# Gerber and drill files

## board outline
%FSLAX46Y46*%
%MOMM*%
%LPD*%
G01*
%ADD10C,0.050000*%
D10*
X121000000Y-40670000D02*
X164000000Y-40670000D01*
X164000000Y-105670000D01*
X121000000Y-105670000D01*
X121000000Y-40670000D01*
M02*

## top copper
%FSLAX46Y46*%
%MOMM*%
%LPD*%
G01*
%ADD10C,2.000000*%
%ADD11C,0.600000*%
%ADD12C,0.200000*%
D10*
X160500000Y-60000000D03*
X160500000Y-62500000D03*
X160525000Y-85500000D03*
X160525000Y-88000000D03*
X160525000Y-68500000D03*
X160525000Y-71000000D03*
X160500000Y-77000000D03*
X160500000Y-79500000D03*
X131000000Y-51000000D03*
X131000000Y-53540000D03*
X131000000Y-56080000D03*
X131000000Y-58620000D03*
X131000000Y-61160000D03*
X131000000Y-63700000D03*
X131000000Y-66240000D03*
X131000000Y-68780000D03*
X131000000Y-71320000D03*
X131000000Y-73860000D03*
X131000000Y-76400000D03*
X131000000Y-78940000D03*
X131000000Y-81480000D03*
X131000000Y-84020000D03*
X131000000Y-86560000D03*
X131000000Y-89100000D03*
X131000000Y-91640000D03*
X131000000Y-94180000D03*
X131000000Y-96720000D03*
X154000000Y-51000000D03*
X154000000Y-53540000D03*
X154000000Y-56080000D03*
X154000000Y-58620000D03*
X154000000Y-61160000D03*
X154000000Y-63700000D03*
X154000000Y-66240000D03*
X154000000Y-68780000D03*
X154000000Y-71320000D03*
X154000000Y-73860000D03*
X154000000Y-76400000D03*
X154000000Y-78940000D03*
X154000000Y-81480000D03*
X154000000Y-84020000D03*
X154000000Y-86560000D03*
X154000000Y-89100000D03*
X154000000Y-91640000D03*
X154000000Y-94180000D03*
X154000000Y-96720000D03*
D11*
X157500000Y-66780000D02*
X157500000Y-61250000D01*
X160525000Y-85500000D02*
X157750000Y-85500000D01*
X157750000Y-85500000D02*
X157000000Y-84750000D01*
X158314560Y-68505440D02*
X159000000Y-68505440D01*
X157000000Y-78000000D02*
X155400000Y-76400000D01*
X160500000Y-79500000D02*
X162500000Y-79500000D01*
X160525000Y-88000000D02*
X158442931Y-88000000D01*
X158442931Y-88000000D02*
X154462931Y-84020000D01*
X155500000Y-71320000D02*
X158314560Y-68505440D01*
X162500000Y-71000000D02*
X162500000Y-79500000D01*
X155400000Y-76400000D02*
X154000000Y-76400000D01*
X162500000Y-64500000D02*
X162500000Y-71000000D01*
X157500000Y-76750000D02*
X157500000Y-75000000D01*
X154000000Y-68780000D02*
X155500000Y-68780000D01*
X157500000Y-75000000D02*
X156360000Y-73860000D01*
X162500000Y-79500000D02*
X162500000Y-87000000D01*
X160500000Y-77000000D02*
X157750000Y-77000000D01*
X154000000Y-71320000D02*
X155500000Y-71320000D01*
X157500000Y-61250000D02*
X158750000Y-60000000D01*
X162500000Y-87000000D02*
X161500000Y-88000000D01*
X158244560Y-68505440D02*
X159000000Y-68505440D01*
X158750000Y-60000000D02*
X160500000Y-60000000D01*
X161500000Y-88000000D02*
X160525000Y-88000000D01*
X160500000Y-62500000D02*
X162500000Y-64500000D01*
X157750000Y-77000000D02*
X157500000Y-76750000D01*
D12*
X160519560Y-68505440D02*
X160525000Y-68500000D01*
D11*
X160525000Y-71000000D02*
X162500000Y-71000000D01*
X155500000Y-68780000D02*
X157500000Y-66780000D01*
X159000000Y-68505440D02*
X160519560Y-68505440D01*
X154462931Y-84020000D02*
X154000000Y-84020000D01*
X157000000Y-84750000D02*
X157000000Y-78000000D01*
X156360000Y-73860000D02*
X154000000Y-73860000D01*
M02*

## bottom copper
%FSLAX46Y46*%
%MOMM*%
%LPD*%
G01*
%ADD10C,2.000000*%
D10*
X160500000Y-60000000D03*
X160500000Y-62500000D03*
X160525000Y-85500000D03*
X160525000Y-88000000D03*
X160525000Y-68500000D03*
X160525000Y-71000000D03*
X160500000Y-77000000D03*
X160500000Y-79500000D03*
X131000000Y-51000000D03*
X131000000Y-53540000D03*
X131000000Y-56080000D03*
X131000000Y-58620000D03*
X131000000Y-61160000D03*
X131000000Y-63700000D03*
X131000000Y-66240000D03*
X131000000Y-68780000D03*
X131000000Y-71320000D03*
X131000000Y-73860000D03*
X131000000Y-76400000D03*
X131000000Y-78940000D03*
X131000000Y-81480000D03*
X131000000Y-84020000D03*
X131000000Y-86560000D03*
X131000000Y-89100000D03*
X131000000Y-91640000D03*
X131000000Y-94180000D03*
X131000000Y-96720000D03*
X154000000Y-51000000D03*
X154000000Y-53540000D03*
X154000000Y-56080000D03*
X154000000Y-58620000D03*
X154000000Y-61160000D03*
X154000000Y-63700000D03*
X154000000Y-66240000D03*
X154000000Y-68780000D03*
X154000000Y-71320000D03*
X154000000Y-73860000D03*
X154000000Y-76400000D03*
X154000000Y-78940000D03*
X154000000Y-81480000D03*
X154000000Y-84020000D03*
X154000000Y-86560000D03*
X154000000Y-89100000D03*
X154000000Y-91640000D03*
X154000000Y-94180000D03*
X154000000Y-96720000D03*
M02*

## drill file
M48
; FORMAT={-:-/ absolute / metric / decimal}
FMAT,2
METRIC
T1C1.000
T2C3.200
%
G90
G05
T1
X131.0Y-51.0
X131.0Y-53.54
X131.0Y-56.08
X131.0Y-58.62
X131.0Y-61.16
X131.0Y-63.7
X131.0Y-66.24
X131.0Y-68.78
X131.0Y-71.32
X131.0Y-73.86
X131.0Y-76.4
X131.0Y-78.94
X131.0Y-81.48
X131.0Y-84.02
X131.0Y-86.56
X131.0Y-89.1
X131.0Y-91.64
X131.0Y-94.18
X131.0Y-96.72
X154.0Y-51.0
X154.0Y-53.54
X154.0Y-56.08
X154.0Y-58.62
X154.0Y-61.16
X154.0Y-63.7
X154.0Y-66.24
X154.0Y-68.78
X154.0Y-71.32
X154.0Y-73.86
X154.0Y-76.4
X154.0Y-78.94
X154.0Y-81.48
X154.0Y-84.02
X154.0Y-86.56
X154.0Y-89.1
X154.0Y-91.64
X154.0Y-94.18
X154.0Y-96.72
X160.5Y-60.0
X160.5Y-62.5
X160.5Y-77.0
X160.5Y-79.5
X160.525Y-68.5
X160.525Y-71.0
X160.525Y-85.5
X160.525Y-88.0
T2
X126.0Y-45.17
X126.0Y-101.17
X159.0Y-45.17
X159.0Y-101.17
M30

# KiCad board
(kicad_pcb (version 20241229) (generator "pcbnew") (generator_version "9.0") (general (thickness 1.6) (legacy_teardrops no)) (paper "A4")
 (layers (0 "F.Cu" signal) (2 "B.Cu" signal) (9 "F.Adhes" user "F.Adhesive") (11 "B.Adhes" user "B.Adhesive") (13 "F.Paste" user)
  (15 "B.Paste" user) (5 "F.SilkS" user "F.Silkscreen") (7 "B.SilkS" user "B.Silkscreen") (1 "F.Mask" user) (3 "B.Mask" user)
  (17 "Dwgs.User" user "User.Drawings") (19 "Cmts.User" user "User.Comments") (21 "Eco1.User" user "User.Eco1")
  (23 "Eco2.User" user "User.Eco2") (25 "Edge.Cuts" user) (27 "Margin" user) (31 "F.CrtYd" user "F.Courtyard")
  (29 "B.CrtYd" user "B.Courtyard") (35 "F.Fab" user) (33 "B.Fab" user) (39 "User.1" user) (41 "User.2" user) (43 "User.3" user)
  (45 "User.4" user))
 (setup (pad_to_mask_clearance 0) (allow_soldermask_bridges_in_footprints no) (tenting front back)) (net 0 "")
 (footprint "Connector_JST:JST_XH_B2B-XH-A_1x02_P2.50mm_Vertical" (layer "F.Cu") (at 160.5 60 -90)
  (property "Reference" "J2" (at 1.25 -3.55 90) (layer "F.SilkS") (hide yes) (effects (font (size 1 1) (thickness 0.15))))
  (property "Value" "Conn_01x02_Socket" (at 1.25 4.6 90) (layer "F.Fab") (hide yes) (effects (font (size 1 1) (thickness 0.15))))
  (pad "1" thru_hole circle (at 0 0 270) (size 2 2) (drill 1) (layers "*.Cu" "*.Mask") (remove_unused_layers no))
  (pad "2" thru_hole circle (at 2.5 0 270) (size 2 2) (drill 1) (layers "*.Cu" "*.Mask") (remove_unused_layers no)))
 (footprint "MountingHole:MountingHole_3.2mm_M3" (layer "F.Cu") (at 126 101.17)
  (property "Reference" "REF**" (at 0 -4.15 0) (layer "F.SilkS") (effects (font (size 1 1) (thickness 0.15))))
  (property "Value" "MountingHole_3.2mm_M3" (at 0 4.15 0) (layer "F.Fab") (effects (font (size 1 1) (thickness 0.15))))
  (pad "" np_thru_hole circle (at 0 0) (size 3.2 3.2) (drill 3.2) (layers "*.Cu" "*.Mask")))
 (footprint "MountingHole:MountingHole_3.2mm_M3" (layer "F.Cu") (at 159 45.17)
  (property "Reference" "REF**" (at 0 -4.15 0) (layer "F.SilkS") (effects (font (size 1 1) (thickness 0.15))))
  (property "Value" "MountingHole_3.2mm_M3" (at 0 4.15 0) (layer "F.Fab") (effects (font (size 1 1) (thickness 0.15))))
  (pad "" np_thru_hole circle (at 0 0) (size 3.2 3.2) (drill 3.2) (layers "*.Cu" "*.Mask")))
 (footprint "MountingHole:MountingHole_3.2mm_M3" (layer "F.Cu") (at 159 101.17)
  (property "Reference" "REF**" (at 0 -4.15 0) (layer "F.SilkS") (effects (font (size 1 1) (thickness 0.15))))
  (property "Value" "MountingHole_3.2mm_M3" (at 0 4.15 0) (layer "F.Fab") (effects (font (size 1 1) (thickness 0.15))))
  (pad "" np_thru_hole circle (at 0 0) (size 3.2 3.2) (drill 3.2) (layers "*.Cu" "*.Mask")))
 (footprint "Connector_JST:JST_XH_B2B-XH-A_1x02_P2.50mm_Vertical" (layer "F.Cu") (at 160.525 85.5 -90)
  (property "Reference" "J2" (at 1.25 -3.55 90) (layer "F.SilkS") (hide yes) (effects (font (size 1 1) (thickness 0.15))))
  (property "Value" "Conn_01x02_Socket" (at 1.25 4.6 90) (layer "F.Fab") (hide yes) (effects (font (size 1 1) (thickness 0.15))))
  (pad "1" thru_hole circle (at 0 0 270) (size 2 2) (drill 1) (layers "*.Cu" "*.Mask") (remove_unused_layers no))
  (pad "2" thru_hole circle (at 2.5 0 270) (size 2 2) (drill 1) (layers "*.Cu" "*.Mask") (remove_unused_layers no)))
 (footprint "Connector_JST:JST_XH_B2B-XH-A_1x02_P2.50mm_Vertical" (layer "F.Cu") (at 160.525 68.5 -90)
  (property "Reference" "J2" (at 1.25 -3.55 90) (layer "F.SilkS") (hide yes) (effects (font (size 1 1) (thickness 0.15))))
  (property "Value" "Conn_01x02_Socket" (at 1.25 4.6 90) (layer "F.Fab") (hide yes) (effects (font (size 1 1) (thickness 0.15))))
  (pad "1" thru_hole circle (at 0 0 270) (size 2 2) (drill 1) (layers "*.Cu" "*.Mask") (remove_unused_layers no))
  (pad "2" thru_hole circle (at 2.5 0 270) (size 2 2) (drill 1) (layers "*.Cu" "*.Mask") (remove_unused_layers no)))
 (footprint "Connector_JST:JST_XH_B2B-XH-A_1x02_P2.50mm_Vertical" (layer "F.Cu") (at 160.5 77 -90)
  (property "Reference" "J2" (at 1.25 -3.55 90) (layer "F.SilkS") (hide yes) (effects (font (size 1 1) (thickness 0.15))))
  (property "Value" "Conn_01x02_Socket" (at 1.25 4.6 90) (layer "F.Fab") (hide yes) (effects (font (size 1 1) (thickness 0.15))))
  (pad "1" thru_hole circle (at 0 0 270) (size 2 2) (drill 1) (layers "*.Cu" "*.Mask") (remove_unused_layers no))
  (pad "2" thru_hole circle (at 2.5 0 270) (size 2 2) (drill 1) (layers "*.Cu" "*.Mask") (remove_unused_layers no)))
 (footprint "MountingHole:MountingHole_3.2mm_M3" (layer "F.Cu") (at 126 45.17)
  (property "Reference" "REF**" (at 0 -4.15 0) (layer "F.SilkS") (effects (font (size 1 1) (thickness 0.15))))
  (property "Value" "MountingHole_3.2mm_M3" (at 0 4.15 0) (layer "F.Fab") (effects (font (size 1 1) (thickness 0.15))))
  (pad "" np_thru_hole circle (at 0 0) (size 3.2 3.2) (drill 3.2) (layers "*.Cu" "*.Mask")))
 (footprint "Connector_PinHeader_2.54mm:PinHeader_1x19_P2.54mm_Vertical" (layer "B.Cu") (at 131 51 180)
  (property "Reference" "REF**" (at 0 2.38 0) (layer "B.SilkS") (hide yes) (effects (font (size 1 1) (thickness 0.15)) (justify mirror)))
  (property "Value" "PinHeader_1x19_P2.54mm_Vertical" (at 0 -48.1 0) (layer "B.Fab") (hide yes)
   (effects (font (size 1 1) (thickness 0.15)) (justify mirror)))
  (pad "1" thru_hole circle (at 0 0 180) (size 2 2) (drill 1) (layers "*.Cu" "*.Mask") (remove_unused_layers no))
  (pad "2" thru_hole circle (at 0 -2.54 180) (size 2 2) (drill 1) (layers "*.Cu" "*.Mask") (remove_unused_layers no))
  (pad "3" thru_hole circle (at 0 -5.08 180) (size 2 2) (drill 1) (layers "*.Cu" "*.Mask") (remove_unused_layers no))
  (pad "4" thru_hole circle (at 0 -7.62 180) (size 2 2) (drill 1) (layers "*.Cu" "*.Mask") (remove_unused_layers no))
  (pad "5" thru_hole circle (at 0 -10.16 180) (size 2 2) (drill 1) (layers "*.Cu" "*.Mask") (remove_unused_layers no))
  (pad "6" thru_hole circle (at 0 -12.7 180) (size 2 2) (drill 1) (layers "*.Cu" "*.Mask") (remove_unused_layers no))
  (pad "7" thru_hole circle (at 0 -15.24 180) (size 2 2) (drill 1) (layers "*.Cu" "*.Mask") (remove_unused_layers no))
  (pad "8" thru_hole circle (at 0 -17.78 180) (size 2 2) (drill 1) (layers "*.Cu" "*.Mask") (remove_unused_layers no))
  (pad "9" thru_hole circle (at 0 -20.32 180) (size 2 2) (drill 1) (layers "*.Cu" "*.Mask") (remove_unused_layers no))
  (pad "10" thru_hole circle (at 0 -22.86 180) (size 2 2) (drill 1) (layers "*.Cu" "*.Mask") (remove_unused_layers no))
  (pad "11" thru_hole circle (at 0 -25.4 180) (size 2 2) (drill 1) (layers "*.Cu" "*.Mask") (remove_unused_layers no))
  (pad "12" thru_hole circle (at 0 -27.94 180) (size 2 2) (drill 1) (layers "*.Cu" "*.Mask") (remove_unused_layers no))
  (pad "13" thru_hole circle (at 0 -30.48 180) (size 2 2) (drill 1) (layers "*.Cu" "*.Mask") (remove_unused_layers no))
  (pad "14" thru_hole circle (at 0 -33.02 180) (size 2 2) (drill 1) (layers "*.Cu" "*.Mask") (remove_unused_layers no))
  (pad "15" thru_hole circle (at 0 -35.56 180) (size 2 2) (drill 1) (layers "*.Cu" "*.Mask") (remove_unused_layers no))
  (pad "16" thru_hole circle (at 0 -38.1 180) (size 2 2) (drill 1) (layers "*.Cu" "*.Mask") (remove_unused_layers no))
  (pad "17" thru_hole circle (at 0 -40.64 180) (size 2 2) (drill 1) (layers "*.Cu" "*.Mask") (remove_unused_layers no))
  (pad "18" thru_hole circle (at 0 -43.18 180) (size 2 2) (drill 1) (layers "*.Cu" "*.Mask") (remove_unused_layers no))
  (pad "19" thru_hole circle (at 0 -45.72 180) (size 2 2) (drill 1) (layers "*.Cu" "*.Mask") (remove_unused_layers no)))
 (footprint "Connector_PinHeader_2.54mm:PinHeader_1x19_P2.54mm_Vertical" (layer "B.Cu") (at 154 51 180)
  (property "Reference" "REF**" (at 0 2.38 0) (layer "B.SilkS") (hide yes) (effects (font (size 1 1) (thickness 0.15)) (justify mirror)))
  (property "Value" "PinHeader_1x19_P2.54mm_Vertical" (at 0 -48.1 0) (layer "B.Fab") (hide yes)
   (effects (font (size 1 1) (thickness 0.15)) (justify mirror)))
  (pad "1" thru_hole circle (at 0 0 180) (size 2 2) (drill 1) (layers "*.Cu" "*.Mask") (remove_unused_layers no))
  (pad "2" thru_hole circle (at 0 -2.54 180) (size 2 2) (drill 1) (layers "*.Cu" "*.Mask") (remove_unused_layers no))
  (pad "3" thru_hole circle (at 0 -5.08 180) (size 2 2) (drill 1) (layers "*.Cu" "*.Mask") (remove_unused_layers no))
  (pad "4" thru_hole circle (at 0 -7.62 180) (size 2 2) (drill 1) (layers "*.Cu" "*.Mask") (remove_unused_layers no))
  (pad "5" thru_hole circle (at 0 -10.16 180) (size 2 2) (drill 1) (layers "*.Cu" "*.Mask") (remove_unused_layers no))
  (pad "6" thru_hole circle (at 0 -12.7 180) (size 2 2) (drill 1) (layers "*.Cu" "*.Mask") (remove_unused_layers no))
  (pad "7" thru_hole circle (at 0 -15.24 180) (size 2 2) (drill 1) (layers "*.Cu" "*.Mask") (remove_unused_layers no))
  (pad "8" thru_hole circle (at 0 -17.78 180) (size 2 2) (drill 1) (layers "*.Cu" "*.Mask") (remove_unused_layers no))
  (pad "9" thru_hole circle (at 0 -20.32 180) (size 2 2) (drill 1) (layers "*.Cu" "*.Mask") (remove_unused_layers no))
  (pad "10" thru_hole circle (at 0 -22.86 180) (size 2 2) (drill 1) (layers "*.Cu" "*.Mask") (remove_unused_layers no))
  (pad "11" thru_hole circle (at 0 -25.4 180) (size 2 2) (drill 1) (layers "*.Cu" "*.Mask") (remove_unused_layers no))
  (pad "12" thru_hole circle (at 0 -27.94 180) (size 2 2) (drill 1) (layers "*.Cu" "*.Mask") (remove_unused_layers no))
  (pad "13" thru_hole circle (at 0 -30.48 180) (size 2 2) (drill 1) (layers "*.Cu" "*.Mask") (remove_unused_layers no))
  (pad "14" thru_hole circle (at 0 -33.02 180) (size 2 2) (drill 1) (layers "*.Cu" "*.Mask") (remove_unused_layers no))
  (pad "15" thru_hole circle (at 0 -35.56 180) (size 2 2) (drill 1) (layers "*.Cu" "*.Mask") (remove_unused_layers no))
  (pad "16" thru_hole circle (at 0 -38.1 180) (size 2 2) (drill 1) (layers "*.Cu" "*.Mask") (remove_unused_layers no))
  (pad "17" thru_hole circle (at 0 -40.64 180) (size 2 2) (drill 1) (layers "*.Cu" "*.Mask") (remove_unused_layers no))
  (pad "18" thru_hole circle (at 0 -43.18 180) (size 2 2) (drill 1) (layers "*.Cu" "*.Mask") (remove_unused_layers no))
  (pad "19" thru_hole circle (at 0 -45.72 180) (size 2 2) (drill 1) (layers "*.Cu" "*.Mask") (remove_unused_layers no)))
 (gr_rect (start 121 40.67) (end 164 105.67) (stroke (width 0.05) (type default)) (fill no) (layer "Edge.Cuts"))
 (segment (start 157.5 66.78) (end 157.5 61.25) (width 0.6) (layer "F.Cu") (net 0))
 (segment (start 160.525 85.5) (end 157.75 85.5) (width 0.6) (layer "F.Cu") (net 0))
 (segment (start 157.75 85.5) (end 157 84.75) (width 0.6) (layer "F.Cu") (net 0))
 (segment (start 158.31456 68.50544) (end 159 68.50544) (width 0.6) (layer "F.Cu") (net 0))
 (segment (start 157 78) (end 155.4 76.4) (width 0.6) (layer "F.Cu") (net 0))
 (segment (start 160.5 79.5) (end 162.5 79.5) (width 0.6) (layer "F.Cu") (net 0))
 (segment (start 160.525 88) (end 158.442931 88) (width 0.6) (layer "F.Cu") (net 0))
 (segment (start 158.442931 88) (end 154.462931 84.02) (width 0.6) (layer "F.Cu") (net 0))
 (segment (start 155.5 71.32) (end 158.31456 68.50544) (width 0.6) (layer "F.Cu") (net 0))
 (segment (start 162.5 71) (end 162.5 79.5) (width 0.6) (layer "F.Cu") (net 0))
 (segment (start 155.4 76.4) (end 154 76.4) (width 0.6) (layer "F.Cu") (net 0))
 (segment (start 162.5 64.5) (end 162.5 71) (width 0.6) (layer "F.Cu") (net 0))
 (segment (start 157.5 76.75) (end 157.5 75) (width 0.6) (layer "F.Cu") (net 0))
 (segment (start 154 68.78) (end 155.5 68.78) (width 0.6) (layer "F.Cu") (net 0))
 (segment (start 157.5 75) (end 156.36 73.86) (width 0.6) (layer "F.Cu") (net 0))
 (segment (start 162.5 79.5) (end 162.5 87) (width 0.6) (layer "F.Cu") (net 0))
 (segment (start 160.5 77) (end 157.75 77) (width 0.6) (layer "F.Cu") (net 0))
 (segment (start 154 71.32) (end 155.5 71.32) (width 0.6) (layer "F.Cu") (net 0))
 (segment (start 157.5 61.25) (end 158.75 60) (width 0.6) (layer "F.Cu") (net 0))
 (segment (start 162.5 87) (end 161.5 88) (width 0.6) (layer "F.Cu") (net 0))
 (segment (start 158.24456 68.50544) (end 159 68.50544) (width 0.6) (layer "F.Cu") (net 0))
 (segment (start 158.75 60) (end 160.5 60) (width 0.6) (layer "F.Cu") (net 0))
 (segment (start 161.5 88) (end 160.525 88) (width 0.6) (layer "F.Cu") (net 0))
 (segment (start 160.5 62.5) (end 162.5 64.5) (width 0.6) (layer "F.Cu") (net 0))
 (segment (start 157.75 77) (end 157.5 76.75) (width 0.6) (layer "F.Cu") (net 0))
 (segment (start 160.51956 68.50544) (end 160.525 68.5) (width 0.2) (layer "F.Cu") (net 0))
 (segment (start 160.525 71) (end 162.5 71) (width 0.6) (layer "F.Cu") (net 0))
 (segment (start 155.5 68.78) (end 157.5 66.78) (width 0.6) (layer "F.Cu") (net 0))
 (segment (start 159 68.50544) (end 160.51956 68.50544) (width 0.6) (layer "F.Cu") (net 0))
 (segment (start 154.462931 84.02) (end 154 84.02) (width 0.6) (layer "F.Cu") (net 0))
 (segment (start 157 84.75) (end 157 78) (width 0.6) (layer "F.Cu") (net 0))
 (segment (start 156.36 73.86) (end 154 73.86) (width 0.6) (layer "F.Cu") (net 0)))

